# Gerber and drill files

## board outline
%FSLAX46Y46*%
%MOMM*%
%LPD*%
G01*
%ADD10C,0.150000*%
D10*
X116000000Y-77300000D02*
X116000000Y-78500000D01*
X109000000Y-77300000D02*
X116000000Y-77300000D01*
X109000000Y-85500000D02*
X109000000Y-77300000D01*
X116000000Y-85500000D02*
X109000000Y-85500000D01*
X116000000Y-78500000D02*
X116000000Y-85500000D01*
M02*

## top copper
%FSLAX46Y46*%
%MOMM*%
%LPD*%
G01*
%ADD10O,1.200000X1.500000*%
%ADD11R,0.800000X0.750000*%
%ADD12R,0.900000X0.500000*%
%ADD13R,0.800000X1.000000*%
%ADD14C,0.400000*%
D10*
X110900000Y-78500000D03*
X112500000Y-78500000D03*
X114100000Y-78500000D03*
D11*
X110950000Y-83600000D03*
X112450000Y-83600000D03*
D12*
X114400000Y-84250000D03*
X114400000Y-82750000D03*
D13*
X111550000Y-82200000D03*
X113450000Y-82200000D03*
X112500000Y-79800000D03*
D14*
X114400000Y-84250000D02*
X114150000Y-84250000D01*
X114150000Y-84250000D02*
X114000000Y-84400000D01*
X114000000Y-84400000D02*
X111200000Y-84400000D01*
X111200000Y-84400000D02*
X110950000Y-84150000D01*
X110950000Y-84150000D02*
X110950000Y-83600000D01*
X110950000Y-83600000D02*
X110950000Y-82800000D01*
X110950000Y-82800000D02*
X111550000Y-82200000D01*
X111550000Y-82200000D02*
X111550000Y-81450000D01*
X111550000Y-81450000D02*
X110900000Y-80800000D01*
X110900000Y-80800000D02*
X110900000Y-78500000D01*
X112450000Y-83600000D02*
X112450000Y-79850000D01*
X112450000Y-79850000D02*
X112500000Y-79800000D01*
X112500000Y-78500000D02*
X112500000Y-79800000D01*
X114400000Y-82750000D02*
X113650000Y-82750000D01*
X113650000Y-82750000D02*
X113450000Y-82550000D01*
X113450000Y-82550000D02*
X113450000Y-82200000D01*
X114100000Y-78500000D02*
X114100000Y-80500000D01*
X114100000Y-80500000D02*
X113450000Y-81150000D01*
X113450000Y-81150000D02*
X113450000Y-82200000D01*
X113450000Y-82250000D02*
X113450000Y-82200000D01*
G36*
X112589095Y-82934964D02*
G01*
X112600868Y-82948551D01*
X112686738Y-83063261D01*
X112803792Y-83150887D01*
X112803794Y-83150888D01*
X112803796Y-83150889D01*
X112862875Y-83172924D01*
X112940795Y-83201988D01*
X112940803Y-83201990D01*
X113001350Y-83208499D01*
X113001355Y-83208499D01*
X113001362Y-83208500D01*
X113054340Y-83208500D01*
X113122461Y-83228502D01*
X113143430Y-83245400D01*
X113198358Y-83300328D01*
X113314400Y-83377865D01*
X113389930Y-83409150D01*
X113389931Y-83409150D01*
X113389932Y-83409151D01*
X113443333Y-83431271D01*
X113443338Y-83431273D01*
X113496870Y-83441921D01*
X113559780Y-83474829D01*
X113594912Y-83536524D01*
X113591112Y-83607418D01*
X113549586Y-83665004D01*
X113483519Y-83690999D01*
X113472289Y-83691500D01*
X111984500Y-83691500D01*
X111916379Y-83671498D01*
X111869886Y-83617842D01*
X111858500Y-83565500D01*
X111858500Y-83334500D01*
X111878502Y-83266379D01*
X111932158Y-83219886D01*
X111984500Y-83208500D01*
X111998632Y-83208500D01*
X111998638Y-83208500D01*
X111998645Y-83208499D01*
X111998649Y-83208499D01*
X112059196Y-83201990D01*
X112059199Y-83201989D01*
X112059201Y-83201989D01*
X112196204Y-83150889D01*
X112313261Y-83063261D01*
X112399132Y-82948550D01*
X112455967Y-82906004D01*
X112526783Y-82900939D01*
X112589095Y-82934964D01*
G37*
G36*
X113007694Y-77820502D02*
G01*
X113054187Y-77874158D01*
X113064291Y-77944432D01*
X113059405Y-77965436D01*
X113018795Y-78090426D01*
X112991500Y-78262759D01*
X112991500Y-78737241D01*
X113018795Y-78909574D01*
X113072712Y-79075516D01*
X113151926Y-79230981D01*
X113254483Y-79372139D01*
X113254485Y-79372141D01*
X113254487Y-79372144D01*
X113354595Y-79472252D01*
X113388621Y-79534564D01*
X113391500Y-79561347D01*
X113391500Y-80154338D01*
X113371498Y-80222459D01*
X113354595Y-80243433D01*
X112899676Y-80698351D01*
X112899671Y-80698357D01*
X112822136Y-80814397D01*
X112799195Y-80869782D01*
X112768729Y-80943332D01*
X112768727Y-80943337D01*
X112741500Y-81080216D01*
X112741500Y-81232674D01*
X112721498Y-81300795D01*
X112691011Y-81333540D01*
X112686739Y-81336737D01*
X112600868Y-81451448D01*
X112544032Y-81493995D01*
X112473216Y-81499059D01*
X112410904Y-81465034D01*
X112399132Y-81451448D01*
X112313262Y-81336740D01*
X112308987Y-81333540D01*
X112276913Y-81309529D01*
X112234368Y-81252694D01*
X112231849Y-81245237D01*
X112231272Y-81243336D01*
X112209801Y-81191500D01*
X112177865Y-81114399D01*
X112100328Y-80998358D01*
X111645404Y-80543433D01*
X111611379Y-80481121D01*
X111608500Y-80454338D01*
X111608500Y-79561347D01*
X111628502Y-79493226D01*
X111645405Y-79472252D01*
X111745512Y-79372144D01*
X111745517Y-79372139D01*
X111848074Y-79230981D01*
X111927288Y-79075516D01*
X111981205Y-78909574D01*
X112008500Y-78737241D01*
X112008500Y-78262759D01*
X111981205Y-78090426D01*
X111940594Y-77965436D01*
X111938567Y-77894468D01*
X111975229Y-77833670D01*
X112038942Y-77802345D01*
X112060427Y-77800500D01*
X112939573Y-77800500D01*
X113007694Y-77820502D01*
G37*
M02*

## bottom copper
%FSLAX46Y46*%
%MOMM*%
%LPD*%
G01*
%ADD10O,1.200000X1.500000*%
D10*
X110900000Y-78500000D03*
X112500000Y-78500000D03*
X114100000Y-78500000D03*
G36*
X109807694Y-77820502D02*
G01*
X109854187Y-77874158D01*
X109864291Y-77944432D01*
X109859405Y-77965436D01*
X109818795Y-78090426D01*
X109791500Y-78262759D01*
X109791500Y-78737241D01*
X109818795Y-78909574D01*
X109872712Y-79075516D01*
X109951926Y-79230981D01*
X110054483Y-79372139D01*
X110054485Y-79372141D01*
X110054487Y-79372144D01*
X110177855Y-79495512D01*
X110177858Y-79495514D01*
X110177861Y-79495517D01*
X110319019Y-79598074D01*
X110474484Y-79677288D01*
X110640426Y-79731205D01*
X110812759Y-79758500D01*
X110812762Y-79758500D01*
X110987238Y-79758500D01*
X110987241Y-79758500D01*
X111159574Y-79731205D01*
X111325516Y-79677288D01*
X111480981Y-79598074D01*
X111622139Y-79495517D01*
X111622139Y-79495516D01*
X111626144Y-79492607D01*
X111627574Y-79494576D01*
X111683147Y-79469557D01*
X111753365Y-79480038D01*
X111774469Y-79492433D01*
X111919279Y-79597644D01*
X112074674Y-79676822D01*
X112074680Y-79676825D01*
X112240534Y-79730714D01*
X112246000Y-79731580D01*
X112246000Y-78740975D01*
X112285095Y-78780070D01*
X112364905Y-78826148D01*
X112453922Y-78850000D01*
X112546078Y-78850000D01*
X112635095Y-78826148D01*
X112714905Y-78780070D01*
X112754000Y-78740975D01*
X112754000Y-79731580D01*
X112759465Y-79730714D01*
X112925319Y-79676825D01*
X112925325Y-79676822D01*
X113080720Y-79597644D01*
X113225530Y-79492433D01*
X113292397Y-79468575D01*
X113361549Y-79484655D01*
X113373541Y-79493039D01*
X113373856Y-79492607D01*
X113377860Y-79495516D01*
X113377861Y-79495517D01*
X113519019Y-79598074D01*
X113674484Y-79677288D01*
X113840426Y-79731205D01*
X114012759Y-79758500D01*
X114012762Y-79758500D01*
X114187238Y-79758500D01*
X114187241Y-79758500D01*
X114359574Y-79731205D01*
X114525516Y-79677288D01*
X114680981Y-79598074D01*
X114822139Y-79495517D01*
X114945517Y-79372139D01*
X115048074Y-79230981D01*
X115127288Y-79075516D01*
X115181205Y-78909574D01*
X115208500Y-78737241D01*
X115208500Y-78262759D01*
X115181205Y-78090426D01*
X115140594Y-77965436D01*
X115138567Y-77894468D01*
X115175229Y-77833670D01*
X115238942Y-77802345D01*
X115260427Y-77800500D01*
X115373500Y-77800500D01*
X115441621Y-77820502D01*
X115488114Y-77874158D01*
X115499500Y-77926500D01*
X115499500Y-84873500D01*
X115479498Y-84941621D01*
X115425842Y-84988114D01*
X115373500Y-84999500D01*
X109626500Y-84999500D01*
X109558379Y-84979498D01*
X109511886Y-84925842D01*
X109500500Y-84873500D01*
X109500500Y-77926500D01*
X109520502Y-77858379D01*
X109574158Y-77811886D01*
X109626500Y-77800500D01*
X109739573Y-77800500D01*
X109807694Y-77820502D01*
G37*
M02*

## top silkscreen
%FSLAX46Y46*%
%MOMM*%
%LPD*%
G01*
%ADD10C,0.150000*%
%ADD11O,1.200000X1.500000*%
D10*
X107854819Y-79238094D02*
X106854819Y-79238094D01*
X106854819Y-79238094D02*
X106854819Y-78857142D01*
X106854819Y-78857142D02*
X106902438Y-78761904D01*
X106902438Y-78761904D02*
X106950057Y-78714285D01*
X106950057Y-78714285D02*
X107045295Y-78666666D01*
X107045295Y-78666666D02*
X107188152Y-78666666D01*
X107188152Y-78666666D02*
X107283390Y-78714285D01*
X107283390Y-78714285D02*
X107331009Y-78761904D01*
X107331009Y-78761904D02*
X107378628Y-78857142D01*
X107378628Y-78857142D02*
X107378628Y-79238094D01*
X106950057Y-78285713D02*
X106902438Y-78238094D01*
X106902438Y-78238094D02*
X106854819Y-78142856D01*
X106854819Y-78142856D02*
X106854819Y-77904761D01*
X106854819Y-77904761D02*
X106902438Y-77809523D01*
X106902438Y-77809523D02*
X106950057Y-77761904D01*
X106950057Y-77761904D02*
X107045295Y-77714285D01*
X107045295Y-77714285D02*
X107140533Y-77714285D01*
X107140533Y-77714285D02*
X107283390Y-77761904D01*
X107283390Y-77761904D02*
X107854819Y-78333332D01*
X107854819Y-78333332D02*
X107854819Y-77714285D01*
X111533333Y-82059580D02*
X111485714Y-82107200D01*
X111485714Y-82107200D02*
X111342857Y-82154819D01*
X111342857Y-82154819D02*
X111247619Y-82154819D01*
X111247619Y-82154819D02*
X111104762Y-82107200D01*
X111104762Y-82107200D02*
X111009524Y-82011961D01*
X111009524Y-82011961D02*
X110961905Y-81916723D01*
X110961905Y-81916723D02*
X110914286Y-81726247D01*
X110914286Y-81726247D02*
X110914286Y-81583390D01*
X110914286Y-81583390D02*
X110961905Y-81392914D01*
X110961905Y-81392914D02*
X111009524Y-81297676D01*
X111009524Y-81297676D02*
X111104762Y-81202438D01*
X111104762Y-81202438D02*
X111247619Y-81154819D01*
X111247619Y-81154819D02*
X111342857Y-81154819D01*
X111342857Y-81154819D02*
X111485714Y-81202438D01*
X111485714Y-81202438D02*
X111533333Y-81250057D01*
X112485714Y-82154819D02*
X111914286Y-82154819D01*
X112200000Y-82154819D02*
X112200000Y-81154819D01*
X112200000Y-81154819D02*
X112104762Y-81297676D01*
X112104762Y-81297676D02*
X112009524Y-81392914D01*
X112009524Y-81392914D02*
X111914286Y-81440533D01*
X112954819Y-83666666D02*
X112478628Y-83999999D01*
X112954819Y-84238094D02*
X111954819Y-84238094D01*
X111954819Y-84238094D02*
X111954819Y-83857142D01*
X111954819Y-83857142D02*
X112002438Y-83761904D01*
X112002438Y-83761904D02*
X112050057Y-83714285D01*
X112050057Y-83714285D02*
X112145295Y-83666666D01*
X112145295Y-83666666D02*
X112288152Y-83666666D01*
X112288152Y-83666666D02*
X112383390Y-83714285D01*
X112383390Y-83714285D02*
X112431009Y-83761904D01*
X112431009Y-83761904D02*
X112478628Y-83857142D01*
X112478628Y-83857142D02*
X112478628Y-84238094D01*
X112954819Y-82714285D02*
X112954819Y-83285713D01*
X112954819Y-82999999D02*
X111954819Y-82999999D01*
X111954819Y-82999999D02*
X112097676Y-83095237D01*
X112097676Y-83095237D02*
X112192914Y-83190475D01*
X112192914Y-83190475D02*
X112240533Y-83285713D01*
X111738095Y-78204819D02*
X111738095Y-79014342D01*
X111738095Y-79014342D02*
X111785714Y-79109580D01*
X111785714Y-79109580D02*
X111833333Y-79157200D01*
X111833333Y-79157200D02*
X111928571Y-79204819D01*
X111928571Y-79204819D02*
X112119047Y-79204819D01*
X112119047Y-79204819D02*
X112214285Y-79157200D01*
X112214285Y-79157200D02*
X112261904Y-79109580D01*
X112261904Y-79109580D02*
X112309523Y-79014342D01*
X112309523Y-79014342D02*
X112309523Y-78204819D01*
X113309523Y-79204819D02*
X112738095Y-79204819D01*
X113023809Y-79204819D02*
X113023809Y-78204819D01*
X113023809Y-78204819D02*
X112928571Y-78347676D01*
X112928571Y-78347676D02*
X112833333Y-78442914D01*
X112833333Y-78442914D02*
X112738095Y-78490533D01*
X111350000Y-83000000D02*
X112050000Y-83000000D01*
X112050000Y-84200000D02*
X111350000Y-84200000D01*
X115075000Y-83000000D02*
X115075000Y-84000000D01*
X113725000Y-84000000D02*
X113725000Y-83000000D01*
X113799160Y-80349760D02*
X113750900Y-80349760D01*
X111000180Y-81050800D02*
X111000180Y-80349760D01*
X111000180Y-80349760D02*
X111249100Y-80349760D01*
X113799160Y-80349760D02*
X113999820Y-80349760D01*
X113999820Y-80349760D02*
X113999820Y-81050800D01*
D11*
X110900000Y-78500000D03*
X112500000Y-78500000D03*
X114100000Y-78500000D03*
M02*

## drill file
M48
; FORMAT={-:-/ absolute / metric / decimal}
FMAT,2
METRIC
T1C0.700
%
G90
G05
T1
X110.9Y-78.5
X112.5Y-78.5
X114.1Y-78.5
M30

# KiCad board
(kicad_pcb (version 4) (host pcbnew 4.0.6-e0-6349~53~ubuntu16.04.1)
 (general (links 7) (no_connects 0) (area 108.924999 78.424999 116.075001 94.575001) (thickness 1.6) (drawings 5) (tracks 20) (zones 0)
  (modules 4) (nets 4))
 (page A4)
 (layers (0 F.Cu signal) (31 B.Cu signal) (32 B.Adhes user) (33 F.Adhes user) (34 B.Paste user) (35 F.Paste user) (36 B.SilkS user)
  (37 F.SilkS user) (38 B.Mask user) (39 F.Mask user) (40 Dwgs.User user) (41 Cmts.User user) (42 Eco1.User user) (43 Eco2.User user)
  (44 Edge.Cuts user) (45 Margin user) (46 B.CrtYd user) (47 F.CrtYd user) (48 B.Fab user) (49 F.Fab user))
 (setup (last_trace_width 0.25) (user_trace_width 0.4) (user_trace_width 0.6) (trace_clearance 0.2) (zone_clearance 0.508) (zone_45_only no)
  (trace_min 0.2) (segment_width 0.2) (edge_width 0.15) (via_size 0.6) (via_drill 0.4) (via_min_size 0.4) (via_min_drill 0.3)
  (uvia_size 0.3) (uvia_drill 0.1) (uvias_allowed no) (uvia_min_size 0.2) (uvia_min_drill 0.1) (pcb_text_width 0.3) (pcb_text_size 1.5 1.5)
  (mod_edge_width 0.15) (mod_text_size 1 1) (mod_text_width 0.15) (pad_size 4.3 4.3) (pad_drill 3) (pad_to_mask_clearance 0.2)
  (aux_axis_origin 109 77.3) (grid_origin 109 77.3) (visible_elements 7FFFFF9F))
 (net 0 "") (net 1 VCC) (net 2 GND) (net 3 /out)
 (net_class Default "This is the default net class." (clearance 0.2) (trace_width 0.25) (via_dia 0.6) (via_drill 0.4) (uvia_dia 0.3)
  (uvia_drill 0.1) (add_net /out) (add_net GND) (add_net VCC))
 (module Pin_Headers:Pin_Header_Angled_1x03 (layer F.Cu) (at 112.5 78.5 90)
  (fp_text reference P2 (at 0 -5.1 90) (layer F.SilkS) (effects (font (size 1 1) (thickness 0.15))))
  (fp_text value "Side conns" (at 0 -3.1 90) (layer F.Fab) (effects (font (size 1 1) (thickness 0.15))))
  (pad 1 thru_hole oval (at 0 -1.6 90) (size 1.5 1.2) (drill 0.7) (layers *.Cu *.Mask F.SilkS) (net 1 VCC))
  (pad 2 thru_hole oval (at 0 0 90) (size 1.5 1.2) (drill 0.7) (layers *.Cu *.Mask F.SilkS) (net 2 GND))
  (pad 3 thru_hole oval (at 0 1.6 90) (size 1.5 1.2) (drill 0.7) (layers *.Cu *.Mask F.SilkS) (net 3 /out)))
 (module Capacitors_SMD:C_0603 (layer F.Cu) (at 111.7 83.6)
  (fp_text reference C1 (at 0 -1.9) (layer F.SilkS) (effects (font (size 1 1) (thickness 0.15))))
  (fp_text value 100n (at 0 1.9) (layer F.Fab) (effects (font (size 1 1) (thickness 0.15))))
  (fp_line (start -0.35 -0.6) (end 0.35 -0.6) (layer F.SilkS) (width 0.15))
  (fp_line (start 0.35 0.6) (end -0.35 0.6) (layer F.SilkS) (width 0.15))
  (pad 1 smd rect (at -0.75 0) (size 0.8 0.75) (layers F.Cu F.Paste F.Mask) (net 1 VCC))
  (pad 2 smd rect (at 0.75 0) (size 0.8 0.75) (layers F.Cu F.Paste F.Mask) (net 2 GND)))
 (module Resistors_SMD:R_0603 (layer F.Cu) (at 114.4 83.5 90)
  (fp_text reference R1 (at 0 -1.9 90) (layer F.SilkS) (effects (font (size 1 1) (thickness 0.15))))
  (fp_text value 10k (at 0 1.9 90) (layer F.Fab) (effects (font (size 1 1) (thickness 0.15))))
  (fp_line (start 0.5 0.675) (end -0.5 0.675) (layer F.SilkS) (width 0.15))
  (fp_line (start -0.5 -0.675) (end 0.5 -0.675) (layer F.SilkS) (width 0.15))
  (pad 1 smd rect (at -0.75 0 90) (size 0.5 0.9) (layers F.Cu F.Paste F.Mask) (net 1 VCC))
  (pad 2 smd rect (at 0.75 0 90) (size 0.5 0.9) (layers F.Cu F.Paste F.Mask) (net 3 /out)))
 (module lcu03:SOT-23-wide (layer F.Cu) (at 112.5 81)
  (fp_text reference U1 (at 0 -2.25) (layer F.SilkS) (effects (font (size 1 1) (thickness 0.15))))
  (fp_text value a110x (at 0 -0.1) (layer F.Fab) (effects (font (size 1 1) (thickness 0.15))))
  (fp_line (start 1.29916 -0.65024) (end 1.2509 -0.65024) (layer F.SilkS) (width 0.15))
  (fp_line (start -1.49982 0.0508) (end -1.49982 -0.65024) (layer F.SilkS) (width 0.15))
  (fp_line (start -1.49982 -0.65024) (end -1.2509 -0.65024) (layer F.SilkS) (width 0.15))
  (fp_line (start 1.29916 -0.65024) (end 1.49982 -0.65024) (layer F.SilkS) (width 0.15))
  (fp_line (start 1.49982 -0.65024) (end 1.49982 0.0508) (layer F.SilkS) (width 0.15))
  (pad 1 smd rect (at -0.95 1.2) (size 0.8 1) (layers F.Cu F.Paste F.Mask) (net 1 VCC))
  (pad 2 smd rect (at 0.95 1.2) (size 0.8 1) (layers F.Cu F.Paste F.Mask) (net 3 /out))
  (pad 3 smd rect (at 0 -1.2) (size 0.8 1) (layers F.Cu F.Paste F.Mask) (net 2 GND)))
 (gr_line (start 116 77.3) (end 116 78.5) (angle 90) (layer Edge.Cuts) (width 0.15))
 (gr_line (start 109 77.3) (end 116 77.3) (angle 90) (layer Edge.Cuts) (width 0.15))
 (gr_line (start 109 85.5) (end 109 77.3) (angle 90) (layer Edge.Cuts) (width 0.15))
 (gr_line (start 116 85.5) (end 109 85.5) (angle 90) (layer Edge.Cuts) (width 0.15))
 (gr_line (start 116 78.5) (end 116 85.5) (angle 90) (layer Edge.Cuts) (width 0.15))
 (segment (start 114.4 84.25) (end 114.15 84.25) (width 0.4) (layer F.Cu) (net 1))
 (segment (start 114.15 84.25) (end 114 84.4) (width 0.4) (layer F.Cu) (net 1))
 (segment (start 114 84.4) (end 111.2 84.4) (width 0.4) (layer F.Cu) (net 1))
 (segment (start 111.2 84.4) (end 110.95 84.15) (width 0.4) (layer F.Cu) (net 1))
 (segment (start 110.95 84.15) (end 110.95 83.6) (width 0.4) (layer F.Cu) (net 1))
 (segment (start 110.95 83.6) (end 110.95 82.8) (width 0.4) (layer F.Cu) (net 1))
 (segment (start 110.95 82.8) (end 111.55 82.2) (width 0.4) (layer F.Cu) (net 1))
 (segment (start 111.55 82.2) (end 111.55 81.45) (width 0.4) (layer F.Cu) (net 1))
 (segment (start 111.55 81.45) (end 110.9 80.8) (width 0.4) (layer F.Cu) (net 1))
 (segment (start 110.9 80.8) (end 110.9 78.5) (width 0.4) (layer F.Cu) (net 1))
 (segment (start 112.45 83.6) (end 112.45 79.85) (width 0.4) (layer F.Cu) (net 2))
 (segment (start 112.45 79.85) (end 112.5 79.8) (width 0.4) (layer F.Cu) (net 2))
 (segment (start 112.5 78.5) (end 112.5 79.8) (width 0.4) (layer F.Cu) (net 2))
 (segment (start 114.4 82.75) (end 113.65 82.75) (width 0.4) (layer F.Cu) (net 3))
 (segment (start 113.65 82.75) (end 113.45 82.55) (width 0.4) (layer F.Cu) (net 3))
 (segment (start 113.45 82.55) (end 113.45 82.2) (width 0.4) (layer F.Cu) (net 3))
 (segment (start 114.1 78.5) (end 114.1 80.5) (width 0.4) (layer F.Cu) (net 3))
 (segment (start 114.1 80.5) (end 113.45 81.15) (width 0.4) (layer F.Cu) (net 3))
 (segment (start 113.45 81.15) (end 113.45 82.2) (width 0.4) (layer F.Cu) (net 3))
 (segment (start 113.45 82.25) (end 113.45 82.2) (width 0.4) (layer F.Cu) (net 3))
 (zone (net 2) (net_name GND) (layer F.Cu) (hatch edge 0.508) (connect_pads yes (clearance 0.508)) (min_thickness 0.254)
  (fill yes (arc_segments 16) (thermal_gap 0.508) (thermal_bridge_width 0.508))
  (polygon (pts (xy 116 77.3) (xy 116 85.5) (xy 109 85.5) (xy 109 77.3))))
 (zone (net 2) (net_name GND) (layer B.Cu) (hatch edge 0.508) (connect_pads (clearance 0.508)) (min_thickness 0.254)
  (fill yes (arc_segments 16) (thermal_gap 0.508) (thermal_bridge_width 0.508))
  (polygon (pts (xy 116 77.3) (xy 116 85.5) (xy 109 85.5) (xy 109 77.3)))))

